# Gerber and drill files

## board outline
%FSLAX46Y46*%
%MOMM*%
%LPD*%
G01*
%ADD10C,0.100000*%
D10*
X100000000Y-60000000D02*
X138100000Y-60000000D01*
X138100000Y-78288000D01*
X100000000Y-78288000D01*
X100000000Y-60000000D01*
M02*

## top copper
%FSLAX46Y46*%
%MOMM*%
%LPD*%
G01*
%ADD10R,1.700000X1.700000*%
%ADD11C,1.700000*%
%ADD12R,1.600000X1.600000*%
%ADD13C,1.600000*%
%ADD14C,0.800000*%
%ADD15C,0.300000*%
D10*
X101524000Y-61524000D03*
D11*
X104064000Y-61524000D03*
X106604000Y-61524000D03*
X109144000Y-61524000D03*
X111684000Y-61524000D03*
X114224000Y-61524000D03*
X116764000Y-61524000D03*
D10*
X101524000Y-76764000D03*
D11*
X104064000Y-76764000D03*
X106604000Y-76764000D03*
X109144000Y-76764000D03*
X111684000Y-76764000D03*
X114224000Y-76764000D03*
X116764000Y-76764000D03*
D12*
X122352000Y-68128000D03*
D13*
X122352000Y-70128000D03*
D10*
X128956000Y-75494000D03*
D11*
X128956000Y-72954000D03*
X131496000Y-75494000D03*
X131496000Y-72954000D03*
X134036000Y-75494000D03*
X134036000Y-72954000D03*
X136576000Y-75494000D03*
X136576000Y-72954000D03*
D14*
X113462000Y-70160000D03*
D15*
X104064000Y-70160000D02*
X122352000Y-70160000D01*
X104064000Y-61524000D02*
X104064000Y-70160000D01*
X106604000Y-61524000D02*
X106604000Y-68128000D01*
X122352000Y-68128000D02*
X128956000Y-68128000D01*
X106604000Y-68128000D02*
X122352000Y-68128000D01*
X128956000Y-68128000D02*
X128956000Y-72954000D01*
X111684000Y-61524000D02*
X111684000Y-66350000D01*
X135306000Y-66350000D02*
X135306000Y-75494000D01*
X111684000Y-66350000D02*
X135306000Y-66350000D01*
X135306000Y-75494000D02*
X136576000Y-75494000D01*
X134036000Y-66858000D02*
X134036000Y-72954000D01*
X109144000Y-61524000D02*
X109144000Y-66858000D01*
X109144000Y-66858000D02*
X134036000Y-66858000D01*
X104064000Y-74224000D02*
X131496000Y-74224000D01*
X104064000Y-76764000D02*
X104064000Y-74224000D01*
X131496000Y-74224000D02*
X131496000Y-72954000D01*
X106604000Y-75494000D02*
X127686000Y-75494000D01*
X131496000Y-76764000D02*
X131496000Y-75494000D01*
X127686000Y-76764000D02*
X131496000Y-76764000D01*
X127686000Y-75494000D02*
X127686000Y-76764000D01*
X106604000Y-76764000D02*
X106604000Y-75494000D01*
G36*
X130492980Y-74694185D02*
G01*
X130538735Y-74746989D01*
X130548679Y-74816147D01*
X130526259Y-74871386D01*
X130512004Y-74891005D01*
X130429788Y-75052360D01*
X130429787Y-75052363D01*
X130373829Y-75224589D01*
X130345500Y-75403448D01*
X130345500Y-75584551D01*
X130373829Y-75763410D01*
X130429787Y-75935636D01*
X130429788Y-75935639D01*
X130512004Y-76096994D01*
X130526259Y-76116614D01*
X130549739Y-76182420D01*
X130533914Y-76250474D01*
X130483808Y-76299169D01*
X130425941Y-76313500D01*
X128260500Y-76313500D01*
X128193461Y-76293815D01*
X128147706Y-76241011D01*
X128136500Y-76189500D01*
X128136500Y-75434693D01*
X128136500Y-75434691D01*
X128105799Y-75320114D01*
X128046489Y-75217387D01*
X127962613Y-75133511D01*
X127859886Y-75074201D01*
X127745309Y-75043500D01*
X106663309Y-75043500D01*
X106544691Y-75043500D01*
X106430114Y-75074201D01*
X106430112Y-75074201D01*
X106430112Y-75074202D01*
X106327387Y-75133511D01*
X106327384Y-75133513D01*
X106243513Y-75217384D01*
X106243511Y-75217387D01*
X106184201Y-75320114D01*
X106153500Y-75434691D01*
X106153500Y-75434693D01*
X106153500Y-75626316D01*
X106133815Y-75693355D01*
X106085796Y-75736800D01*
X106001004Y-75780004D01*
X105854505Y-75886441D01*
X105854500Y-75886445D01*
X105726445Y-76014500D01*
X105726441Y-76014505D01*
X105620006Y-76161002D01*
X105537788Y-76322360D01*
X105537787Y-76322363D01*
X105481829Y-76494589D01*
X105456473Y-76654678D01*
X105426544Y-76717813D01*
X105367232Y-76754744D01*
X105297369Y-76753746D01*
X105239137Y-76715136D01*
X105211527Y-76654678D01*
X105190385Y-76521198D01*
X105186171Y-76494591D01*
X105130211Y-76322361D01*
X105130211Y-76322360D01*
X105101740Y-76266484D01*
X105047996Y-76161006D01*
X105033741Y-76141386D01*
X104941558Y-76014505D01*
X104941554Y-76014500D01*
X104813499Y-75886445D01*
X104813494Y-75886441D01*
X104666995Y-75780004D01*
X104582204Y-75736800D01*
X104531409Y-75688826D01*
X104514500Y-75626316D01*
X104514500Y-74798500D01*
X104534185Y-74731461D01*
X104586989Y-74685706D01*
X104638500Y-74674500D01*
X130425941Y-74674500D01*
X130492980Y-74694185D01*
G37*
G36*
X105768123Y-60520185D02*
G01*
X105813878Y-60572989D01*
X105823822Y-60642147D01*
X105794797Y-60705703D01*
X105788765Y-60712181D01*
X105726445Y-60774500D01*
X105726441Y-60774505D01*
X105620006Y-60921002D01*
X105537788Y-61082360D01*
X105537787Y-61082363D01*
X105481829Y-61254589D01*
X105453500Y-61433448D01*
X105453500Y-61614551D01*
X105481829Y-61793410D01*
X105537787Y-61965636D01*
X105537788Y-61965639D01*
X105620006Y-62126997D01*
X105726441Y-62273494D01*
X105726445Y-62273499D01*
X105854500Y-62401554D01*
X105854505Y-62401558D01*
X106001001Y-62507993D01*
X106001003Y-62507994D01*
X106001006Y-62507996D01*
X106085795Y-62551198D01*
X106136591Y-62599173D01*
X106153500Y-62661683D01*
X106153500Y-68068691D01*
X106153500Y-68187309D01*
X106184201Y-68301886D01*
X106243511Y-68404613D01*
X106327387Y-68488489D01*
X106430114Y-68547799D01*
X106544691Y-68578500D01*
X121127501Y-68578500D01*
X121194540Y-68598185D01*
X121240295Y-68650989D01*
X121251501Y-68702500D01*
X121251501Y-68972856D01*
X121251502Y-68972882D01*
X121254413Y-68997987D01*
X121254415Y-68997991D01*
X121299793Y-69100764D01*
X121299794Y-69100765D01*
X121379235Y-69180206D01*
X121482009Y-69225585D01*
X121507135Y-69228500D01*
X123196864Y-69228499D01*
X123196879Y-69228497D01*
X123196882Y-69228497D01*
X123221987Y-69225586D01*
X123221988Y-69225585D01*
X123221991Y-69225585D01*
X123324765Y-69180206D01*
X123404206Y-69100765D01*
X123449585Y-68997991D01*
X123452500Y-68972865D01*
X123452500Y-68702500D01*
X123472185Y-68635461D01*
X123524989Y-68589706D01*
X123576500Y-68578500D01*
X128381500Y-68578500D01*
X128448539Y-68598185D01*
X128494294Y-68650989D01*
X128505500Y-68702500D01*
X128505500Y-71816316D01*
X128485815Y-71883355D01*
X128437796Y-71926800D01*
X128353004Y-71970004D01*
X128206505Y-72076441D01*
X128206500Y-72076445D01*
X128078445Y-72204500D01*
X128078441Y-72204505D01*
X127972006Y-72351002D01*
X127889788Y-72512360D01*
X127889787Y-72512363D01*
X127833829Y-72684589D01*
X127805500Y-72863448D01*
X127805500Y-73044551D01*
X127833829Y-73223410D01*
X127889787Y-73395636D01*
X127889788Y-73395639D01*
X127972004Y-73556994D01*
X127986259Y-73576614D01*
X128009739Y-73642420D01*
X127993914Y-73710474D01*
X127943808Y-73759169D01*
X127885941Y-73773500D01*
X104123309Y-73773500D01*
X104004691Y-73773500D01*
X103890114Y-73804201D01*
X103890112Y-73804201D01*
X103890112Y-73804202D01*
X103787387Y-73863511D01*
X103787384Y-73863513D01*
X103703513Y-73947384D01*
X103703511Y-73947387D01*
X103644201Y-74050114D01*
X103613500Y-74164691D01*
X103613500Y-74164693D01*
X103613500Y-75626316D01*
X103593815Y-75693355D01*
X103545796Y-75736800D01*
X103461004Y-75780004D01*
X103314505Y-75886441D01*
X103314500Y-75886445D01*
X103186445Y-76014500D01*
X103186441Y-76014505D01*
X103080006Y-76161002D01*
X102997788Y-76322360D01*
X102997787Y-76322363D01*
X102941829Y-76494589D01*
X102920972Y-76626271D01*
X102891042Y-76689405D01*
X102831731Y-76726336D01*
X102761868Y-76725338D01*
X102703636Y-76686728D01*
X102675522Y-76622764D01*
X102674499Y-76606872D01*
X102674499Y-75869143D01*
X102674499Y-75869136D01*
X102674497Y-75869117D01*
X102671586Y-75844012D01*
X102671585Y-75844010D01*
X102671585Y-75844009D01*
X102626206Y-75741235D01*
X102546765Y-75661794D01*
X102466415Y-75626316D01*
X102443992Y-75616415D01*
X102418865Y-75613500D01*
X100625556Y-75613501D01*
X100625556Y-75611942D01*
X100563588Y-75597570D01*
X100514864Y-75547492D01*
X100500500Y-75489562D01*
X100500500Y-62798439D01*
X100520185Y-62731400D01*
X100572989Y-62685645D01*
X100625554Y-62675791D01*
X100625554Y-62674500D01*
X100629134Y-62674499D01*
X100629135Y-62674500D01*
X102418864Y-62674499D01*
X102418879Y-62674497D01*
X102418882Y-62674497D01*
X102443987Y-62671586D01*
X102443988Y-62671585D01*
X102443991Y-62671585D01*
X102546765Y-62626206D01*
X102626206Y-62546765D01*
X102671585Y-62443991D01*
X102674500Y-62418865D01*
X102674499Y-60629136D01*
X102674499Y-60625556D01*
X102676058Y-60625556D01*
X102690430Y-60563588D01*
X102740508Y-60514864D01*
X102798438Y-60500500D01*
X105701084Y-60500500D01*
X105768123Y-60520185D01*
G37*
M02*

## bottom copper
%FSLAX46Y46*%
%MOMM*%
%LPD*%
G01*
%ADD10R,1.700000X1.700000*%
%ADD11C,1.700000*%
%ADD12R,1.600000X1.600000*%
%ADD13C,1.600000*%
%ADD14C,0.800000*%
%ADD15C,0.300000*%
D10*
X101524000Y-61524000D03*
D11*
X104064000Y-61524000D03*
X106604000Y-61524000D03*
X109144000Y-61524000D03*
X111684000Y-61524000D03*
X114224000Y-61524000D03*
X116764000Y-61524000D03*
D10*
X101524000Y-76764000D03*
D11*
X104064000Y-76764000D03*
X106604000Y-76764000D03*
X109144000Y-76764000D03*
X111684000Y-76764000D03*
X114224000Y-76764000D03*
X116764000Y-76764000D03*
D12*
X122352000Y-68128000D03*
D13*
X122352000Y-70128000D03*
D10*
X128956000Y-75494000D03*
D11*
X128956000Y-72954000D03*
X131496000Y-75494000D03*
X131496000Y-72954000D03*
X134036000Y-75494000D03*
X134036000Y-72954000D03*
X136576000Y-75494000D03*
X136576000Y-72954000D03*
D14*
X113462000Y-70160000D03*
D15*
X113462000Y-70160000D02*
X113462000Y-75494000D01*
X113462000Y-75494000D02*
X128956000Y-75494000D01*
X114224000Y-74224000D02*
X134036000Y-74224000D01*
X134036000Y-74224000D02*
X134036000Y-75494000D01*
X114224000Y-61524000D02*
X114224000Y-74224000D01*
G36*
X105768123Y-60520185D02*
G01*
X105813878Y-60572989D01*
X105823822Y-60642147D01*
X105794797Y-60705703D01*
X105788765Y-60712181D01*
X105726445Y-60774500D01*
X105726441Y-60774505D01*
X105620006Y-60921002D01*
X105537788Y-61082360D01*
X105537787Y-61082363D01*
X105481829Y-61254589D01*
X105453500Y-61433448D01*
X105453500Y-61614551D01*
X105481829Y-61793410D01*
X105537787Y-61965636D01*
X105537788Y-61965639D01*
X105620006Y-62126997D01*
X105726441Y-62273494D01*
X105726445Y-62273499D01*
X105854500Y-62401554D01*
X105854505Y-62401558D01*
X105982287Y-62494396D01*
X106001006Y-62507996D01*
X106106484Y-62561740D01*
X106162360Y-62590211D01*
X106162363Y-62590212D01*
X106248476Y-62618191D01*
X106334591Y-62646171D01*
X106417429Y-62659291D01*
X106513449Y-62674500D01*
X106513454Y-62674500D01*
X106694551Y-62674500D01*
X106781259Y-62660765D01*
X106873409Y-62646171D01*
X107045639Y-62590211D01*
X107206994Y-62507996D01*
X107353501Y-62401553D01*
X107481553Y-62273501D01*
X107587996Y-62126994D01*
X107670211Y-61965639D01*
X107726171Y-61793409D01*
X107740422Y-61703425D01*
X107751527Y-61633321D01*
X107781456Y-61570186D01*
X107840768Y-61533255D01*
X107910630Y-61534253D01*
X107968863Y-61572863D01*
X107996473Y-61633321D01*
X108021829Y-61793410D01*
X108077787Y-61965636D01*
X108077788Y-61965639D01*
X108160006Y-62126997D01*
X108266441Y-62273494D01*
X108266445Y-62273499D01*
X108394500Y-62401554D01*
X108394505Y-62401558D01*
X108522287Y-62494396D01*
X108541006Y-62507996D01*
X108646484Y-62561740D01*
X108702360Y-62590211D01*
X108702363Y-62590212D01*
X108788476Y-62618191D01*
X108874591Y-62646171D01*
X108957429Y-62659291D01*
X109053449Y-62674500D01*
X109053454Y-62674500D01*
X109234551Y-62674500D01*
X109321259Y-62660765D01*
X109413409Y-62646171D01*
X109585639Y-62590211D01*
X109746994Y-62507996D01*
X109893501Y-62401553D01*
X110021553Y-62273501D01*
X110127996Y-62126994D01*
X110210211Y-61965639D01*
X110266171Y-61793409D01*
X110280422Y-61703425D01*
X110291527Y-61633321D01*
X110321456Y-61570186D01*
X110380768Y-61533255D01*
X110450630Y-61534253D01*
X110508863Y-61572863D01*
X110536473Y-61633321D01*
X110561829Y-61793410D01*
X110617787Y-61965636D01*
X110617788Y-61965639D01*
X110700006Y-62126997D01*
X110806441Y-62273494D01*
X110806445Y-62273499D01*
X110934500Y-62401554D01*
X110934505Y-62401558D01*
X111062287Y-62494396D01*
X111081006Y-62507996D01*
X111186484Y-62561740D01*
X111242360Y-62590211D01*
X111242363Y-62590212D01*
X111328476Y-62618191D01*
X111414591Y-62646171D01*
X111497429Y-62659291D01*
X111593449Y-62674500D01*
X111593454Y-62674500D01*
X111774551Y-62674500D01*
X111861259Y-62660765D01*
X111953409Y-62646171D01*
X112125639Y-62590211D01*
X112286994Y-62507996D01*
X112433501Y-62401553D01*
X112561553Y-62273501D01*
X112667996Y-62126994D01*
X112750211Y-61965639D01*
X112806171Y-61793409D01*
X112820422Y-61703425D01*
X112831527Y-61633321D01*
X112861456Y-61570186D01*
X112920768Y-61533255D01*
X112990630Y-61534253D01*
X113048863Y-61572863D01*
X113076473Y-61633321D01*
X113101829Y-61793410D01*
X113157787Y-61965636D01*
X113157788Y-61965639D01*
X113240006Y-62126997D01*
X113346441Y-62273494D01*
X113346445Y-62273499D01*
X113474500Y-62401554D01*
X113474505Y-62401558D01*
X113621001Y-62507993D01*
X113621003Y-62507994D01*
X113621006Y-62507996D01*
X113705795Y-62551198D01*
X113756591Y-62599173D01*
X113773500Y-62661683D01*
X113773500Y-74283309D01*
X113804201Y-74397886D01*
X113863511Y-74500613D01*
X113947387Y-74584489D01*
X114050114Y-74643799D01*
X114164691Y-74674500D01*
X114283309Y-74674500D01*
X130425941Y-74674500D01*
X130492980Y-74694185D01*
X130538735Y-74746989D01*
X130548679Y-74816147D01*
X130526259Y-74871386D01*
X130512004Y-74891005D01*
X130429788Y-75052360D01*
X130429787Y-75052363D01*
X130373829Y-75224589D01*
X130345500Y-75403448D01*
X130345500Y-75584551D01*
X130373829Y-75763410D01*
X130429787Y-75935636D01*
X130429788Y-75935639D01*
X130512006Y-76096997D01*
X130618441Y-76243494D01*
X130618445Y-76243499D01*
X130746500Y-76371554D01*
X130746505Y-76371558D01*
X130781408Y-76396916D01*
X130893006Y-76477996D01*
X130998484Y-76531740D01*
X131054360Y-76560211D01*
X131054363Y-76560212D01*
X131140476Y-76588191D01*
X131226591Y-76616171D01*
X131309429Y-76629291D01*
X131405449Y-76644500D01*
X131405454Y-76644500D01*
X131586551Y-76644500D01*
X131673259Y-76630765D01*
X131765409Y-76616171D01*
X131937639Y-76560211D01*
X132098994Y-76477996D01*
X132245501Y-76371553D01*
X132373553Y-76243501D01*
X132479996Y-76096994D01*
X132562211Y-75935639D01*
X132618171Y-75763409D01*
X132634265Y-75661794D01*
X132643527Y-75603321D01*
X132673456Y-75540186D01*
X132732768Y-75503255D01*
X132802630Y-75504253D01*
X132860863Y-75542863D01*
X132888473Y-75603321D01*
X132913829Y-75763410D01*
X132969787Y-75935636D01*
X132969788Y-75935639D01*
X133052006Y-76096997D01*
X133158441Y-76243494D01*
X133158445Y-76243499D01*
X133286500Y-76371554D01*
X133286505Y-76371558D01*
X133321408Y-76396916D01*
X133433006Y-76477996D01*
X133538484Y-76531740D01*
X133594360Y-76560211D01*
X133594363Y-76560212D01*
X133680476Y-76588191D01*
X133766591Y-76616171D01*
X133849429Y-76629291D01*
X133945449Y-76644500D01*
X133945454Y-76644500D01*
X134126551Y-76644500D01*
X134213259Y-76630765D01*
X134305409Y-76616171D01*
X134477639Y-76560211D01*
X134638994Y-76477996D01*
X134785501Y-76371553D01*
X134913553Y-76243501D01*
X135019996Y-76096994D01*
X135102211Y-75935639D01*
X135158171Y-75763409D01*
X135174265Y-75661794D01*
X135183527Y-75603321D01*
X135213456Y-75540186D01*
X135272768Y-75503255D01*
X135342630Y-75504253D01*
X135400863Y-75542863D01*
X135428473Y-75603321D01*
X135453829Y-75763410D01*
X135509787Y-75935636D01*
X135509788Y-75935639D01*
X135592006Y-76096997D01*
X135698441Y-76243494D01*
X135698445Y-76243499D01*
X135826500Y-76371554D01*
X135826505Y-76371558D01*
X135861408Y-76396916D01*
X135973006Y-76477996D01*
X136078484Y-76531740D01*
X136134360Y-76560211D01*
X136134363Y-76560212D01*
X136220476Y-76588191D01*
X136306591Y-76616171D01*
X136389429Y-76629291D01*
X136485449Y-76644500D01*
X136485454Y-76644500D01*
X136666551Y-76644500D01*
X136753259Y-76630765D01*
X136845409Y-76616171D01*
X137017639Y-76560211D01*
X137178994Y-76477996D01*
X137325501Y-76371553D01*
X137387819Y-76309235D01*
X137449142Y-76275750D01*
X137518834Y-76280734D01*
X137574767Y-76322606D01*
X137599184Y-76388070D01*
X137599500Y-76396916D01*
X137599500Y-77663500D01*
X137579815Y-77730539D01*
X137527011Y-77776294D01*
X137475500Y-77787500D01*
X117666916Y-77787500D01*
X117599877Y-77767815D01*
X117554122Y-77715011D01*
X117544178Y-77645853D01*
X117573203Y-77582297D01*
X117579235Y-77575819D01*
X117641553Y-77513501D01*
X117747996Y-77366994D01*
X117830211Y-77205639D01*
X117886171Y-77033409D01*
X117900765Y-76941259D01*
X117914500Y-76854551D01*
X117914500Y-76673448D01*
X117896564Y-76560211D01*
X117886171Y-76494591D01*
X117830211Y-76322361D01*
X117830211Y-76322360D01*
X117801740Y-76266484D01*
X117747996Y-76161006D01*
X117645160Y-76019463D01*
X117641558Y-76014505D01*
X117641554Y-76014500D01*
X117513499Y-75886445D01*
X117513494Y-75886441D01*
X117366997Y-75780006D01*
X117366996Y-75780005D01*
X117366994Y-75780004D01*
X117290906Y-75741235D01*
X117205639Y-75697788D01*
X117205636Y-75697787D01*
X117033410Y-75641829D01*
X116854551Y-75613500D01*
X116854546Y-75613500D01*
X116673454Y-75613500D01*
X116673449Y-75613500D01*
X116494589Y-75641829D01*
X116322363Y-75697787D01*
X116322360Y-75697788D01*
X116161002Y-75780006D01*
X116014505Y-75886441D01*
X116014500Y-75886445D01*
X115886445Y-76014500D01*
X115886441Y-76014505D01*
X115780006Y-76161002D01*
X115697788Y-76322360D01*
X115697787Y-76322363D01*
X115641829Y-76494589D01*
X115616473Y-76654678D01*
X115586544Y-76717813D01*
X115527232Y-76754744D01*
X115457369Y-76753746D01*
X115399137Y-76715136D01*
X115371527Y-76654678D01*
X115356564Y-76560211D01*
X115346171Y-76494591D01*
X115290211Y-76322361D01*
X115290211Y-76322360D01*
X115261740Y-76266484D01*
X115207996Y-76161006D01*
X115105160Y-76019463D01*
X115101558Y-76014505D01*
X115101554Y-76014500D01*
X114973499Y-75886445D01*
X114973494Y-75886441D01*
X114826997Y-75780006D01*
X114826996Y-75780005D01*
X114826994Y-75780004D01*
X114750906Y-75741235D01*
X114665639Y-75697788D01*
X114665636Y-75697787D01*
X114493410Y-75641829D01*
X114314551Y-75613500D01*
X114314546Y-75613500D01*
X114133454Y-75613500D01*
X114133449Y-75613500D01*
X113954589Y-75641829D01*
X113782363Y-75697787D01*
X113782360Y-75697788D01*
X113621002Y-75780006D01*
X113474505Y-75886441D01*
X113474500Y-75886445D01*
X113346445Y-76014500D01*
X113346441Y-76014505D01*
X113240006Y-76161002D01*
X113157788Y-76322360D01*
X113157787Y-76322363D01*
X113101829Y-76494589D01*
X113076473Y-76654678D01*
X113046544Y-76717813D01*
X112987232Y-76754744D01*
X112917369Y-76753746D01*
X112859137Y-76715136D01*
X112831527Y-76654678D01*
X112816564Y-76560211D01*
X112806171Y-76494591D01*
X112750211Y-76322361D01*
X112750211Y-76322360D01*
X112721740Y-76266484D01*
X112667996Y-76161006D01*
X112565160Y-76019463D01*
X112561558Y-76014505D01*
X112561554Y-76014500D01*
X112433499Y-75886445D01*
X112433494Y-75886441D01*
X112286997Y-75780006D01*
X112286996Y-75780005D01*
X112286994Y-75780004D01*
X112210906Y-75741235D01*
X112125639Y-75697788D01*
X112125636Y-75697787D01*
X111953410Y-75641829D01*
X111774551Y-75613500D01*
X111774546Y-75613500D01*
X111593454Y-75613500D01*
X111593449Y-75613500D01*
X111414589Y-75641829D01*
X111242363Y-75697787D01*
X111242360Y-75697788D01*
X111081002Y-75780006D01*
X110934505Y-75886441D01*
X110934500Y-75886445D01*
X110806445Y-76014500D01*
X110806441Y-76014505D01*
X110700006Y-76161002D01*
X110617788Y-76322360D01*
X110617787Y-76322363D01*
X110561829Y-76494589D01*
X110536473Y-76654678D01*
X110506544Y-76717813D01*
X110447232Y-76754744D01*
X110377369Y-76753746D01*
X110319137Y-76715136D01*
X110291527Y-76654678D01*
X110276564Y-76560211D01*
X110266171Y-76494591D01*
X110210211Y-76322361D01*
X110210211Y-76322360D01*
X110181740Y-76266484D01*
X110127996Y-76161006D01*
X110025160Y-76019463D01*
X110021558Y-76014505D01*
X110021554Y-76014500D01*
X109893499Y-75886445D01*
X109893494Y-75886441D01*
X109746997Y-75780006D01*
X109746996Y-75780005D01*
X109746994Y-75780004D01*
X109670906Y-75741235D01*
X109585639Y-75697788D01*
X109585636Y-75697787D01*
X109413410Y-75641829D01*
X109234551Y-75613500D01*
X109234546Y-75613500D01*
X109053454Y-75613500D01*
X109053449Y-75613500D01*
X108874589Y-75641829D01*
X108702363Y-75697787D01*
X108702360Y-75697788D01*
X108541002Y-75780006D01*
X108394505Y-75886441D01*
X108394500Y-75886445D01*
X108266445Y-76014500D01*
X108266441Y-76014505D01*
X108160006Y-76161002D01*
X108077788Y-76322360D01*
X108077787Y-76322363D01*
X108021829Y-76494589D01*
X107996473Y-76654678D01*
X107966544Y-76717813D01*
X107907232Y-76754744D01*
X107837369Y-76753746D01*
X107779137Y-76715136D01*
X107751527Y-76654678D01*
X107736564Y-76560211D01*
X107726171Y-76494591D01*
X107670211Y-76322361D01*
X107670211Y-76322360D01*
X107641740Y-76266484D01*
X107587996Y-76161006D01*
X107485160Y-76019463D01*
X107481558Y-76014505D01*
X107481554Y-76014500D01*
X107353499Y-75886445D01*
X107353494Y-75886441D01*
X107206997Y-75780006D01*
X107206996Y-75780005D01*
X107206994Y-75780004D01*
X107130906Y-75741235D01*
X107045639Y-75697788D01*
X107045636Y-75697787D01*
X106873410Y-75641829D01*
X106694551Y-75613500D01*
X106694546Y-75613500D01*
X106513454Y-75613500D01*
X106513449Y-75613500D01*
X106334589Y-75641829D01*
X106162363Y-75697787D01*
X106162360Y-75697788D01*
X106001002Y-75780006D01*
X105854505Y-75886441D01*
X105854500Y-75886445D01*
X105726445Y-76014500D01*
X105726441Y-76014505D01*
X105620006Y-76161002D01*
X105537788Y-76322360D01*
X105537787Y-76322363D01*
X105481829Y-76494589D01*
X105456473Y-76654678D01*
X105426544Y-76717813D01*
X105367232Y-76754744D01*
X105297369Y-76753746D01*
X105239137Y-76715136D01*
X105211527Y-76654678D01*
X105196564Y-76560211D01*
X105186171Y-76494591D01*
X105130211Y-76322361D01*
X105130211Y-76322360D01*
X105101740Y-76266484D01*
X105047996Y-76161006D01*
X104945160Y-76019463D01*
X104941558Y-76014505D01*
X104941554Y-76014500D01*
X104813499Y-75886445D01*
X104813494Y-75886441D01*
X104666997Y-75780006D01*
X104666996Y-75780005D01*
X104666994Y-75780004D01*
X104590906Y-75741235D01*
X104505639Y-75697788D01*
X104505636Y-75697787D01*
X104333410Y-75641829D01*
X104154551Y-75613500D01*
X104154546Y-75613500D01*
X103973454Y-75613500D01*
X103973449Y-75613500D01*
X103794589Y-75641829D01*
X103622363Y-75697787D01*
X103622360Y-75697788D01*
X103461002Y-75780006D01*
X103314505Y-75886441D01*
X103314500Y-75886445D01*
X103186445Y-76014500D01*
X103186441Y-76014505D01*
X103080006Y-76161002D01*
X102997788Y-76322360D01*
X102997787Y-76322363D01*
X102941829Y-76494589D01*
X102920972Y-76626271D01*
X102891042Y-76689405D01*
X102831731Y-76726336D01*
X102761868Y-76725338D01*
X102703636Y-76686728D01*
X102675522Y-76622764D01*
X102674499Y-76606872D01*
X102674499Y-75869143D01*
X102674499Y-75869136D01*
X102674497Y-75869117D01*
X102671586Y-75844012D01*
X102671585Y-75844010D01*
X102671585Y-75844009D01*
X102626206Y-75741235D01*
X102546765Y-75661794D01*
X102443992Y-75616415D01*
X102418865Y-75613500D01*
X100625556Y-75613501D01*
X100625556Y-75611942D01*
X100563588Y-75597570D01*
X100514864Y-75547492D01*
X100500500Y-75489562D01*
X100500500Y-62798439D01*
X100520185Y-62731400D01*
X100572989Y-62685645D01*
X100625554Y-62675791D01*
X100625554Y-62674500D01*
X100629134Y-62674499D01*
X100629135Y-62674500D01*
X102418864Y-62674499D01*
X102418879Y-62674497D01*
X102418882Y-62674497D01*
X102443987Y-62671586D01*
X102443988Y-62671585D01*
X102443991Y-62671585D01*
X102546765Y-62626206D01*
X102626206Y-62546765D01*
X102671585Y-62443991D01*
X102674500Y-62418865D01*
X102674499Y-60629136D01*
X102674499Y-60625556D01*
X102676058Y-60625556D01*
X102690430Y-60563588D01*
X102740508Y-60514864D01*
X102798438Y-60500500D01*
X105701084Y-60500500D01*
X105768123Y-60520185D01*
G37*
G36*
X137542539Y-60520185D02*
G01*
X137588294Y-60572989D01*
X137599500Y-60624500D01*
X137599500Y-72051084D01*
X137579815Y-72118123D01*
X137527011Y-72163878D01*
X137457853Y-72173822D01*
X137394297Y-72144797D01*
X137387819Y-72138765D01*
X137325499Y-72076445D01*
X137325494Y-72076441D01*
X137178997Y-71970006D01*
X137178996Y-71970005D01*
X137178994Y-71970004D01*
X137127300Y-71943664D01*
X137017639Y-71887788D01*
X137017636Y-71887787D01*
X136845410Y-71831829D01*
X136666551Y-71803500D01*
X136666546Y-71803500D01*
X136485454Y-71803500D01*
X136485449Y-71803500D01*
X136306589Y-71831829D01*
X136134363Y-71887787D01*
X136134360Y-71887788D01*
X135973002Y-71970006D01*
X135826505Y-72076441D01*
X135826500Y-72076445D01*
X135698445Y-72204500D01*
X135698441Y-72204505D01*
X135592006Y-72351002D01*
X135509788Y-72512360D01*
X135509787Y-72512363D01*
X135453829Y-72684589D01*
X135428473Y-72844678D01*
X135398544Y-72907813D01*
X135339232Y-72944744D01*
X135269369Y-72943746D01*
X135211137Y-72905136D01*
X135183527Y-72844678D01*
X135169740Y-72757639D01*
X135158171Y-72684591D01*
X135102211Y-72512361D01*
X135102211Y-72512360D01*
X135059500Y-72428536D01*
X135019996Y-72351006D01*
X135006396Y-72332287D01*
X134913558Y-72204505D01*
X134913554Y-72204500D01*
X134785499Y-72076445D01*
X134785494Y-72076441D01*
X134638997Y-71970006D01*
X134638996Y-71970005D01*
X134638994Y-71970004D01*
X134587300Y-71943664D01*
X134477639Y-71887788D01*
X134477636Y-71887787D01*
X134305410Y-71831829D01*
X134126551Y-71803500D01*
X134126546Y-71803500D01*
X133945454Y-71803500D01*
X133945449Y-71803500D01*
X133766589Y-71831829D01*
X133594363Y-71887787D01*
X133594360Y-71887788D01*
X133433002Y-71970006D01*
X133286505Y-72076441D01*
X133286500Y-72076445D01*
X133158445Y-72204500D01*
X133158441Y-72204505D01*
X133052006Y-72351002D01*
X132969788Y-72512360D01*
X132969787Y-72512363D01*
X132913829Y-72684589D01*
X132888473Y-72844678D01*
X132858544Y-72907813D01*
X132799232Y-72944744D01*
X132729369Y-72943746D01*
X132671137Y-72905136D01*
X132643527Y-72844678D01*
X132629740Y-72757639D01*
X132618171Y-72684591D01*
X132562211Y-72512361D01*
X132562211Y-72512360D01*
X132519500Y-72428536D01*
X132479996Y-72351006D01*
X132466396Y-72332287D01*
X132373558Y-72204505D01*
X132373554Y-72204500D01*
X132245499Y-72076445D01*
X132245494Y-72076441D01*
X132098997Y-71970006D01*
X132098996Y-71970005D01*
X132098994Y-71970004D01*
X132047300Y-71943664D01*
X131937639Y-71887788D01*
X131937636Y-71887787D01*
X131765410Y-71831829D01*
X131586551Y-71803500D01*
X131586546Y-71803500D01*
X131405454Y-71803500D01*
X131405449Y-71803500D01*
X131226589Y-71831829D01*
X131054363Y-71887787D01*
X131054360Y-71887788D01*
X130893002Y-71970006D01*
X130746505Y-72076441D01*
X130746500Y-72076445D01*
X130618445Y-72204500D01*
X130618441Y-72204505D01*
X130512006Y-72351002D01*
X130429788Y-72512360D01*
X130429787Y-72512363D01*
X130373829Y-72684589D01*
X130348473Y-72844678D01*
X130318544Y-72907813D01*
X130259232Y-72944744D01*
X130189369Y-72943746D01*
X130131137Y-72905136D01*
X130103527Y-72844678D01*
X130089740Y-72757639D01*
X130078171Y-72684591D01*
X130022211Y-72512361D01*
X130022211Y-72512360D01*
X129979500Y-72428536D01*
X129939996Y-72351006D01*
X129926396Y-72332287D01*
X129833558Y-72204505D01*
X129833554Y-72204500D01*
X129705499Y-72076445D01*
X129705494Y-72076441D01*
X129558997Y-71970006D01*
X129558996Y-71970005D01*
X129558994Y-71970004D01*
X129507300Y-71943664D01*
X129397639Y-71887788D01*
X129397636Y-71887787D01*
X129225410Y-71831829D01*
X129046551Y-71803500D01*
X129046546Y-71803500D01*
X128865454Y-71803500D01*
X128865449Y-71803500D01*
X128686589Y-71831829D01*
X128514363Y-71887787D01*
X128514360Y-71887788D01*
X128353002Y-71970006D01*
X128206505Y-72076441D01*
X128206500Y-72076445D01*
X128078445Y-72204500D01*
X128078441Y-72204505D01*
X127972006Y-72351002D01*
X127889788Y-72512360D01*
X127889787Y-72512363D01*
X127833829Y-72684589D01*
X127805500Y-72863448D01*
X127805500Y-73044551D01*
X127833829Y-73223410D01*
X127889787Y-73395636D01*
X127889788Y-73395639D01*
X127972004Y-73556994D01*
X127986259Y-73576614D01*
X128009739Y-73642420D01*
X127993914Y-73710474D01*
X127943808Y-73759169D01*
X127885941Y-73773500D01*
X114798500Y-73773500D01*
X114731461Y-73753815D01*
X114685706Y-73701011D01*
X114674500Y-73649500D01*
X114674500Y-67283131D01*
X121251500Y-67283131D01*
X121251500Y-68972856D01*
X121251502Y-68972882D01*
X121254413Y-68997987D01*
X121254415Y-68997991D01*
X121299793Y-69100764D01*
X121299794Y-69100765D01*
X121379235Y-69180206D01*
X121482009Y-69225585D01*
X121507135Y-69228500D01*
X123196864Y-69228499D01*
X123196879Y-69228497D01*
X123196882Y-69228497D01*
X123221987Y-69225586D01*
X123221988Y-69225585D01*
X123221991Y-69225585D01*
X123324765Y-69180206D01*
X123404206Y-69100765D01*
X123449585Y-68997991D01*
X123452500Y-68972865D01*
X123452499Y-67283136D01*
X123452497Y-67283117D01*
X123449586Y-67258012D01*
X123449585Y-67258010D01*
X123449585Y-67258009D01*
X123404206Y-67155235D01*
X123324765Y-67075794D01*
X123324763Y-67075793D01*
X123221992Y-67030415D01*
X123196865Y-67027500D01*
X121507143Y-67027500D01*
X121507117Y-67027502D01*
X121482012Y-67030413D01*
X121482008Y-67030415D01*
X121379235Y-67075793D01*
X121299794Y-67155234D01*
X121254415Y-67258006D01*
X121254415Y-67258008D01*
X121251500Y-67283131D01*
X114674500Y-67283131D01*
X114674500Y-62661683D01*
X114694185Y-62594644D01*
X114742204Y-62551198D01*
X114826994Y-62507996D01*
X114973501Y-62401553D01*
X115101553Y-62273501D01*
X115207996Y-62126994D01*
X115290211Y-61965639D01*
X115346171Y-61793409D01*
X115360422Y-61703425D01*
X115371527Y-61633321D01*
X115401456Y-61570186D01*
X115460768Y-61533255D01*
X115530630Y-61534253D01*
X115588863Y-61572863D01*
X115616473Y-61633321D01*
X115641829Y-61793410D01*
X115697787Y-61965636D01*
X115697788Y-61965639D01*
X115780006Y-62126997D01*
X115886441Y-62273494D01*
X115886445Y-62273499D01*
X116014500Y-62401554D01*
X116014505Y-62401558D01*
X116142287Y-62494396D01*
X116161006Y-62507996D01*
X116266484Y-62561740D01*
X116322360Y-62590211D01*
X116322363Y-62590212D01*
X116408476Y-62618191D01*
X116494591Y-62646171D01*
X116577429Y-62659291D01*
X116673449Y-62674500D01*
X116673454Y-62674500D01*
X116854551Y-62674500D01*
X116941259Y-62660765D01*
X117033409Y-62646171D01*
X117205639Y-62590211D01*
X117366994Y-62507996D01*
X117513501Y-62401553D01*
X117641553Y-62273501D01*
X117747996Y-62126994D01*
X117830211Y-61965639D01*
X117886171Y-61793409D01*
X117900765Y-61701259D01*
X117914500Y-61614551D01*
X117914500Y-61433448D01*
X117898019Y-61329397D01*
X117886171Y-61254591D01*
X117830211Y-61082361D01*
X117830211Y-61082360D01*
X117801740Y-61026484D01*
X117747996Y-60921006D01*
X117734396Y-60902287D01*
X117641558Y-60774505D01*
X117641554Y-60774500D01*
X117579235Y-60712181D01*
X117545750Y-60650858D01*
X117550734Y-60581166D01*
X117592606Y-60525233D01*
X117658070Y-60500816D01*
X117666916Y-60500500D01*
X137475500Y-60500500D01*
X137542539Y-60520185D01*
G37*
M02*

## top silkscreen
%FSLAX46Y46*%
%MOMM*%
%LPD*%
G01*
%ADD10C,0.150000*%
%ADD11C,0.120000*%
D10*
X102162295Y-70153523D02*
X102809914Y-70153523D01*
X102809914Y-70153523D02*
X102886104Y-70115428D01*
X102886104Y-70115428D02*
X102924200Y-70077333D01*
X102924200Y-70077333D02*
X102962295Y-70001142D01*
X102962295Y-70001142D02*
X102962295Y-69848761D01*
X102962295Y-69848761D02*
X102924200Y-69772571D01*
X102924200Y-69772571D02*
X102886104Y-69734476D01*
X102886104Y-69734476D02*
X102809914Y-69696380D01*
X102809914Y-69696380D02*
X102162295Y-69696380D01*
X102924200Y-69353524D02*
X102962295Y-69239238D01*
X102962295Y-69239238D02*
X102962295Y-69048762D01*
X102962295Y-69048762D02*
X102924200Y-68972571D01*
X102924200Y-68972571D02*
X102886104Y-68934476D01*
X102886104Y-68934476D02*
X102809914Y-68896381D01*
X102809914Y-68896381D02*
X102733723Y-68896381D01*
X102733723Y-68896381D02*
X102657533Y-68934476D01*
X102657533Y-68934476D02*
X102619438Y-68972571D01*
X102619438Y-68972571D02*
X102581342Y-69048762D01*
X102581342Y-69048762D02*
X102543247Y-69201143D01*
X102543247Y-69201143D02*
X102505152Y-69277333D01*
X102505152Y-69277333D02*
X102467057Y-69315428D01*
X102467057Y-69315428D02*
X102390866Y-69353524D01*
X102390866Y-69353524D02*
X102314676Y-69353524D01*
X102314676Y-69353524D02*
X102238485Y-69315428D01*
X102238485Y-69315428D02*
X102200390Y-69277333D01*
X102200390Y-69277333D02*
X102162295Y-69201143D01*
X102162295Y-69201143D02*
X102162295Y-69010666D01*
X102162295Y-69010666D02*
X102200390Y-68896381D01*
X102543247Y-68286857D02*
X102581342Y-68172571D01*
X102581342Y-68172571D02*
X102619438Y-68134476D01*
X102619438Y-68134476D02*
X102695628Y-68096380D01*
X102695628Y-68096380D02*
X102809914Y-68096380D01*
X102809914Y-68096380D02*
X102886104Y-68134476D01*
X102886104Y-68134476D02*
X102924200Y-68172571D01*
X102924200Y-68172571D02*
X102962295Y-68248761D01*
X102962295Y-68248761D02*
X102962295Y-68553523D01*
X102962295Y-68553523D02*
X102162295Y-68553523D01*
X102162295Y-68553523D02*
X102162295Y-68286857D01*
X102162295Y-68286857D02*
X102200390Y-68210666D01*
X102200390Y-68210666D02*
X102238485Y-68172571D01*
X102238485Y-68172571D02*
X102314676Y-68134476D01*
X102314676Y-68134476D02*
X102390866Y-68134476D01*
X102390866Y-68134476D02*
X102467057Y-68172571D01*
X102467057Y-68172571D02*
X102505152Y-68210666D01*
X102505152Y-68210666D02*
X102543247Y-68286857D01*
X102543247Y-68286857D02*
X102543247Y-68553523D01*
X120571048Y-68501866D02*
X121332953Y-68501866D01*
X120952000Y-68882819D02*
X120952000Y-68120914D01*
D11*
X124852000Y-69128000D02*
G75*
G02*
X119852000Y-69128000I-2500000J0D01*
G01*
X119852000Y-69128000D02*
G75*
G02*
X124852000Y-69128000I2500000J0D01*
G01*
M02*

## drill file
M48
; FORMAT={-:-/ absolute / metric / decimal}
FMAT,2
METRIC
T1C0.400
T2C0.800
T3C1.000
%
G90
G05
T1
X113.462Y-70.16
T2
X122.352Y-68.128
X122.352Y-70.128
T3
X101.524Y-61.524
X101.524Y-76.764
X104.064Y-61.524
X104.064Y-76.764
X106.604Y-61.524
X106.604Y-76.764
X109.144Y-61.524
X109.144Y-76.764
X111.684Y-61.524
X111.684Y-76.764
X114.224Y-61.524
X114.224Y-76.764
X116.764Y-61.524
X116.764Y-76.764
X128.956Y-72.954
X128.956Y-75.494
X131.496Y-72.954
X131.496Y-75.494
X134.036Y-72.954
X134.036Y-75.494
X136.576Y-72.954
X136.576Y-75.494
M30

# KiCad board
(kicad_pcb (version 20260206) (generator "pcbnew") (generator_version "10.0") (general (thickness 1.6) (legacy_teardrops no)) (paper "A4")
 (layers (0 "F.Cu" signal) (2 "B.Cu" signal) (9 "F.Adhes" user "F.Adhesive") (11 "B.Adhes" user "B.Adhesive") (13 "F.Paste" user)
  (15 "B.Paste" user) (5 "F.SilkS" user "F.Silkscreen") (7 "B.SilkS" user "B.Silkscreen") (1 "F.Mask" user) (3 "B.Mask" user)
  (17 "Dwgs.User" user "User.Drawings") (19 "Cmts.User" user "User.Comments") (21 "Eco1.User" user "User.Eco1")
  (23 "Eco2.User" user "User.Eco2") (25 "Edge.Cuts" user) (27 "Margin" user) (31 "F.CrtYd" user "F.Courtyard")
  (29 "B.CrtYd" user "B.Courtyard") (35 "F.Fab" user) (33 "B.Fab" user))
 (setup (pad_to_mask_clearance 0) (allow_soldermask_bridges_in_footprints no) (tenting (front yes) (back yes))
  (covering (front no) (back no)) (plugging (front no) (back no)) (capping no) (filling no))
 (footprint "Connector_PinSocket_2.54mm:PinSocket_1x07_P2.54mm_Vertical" (layer "F.Cu") (at 101.524 61.524)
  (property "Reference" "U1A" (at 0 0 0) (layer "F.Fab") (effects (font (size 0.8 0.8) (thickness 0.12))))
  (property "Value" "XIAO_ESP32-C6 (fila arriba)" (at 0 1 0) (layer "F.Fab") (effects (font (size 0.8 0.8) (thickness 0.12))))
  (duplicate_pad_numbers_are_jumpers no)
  (pad "1" thru_hole rect (at 0 0) (size 1.7 1.7) (drill 1) (layers "*.Cu" "*.Mask") (remove_unused_layers no))
  (pad "2" thru_hole circle (at 2.54 0) (size 1.7 1.7) (drill 1) (layers "*.Cu" "*.Mask") (remove_unused_layers no) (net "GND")
   (zone_connect 2))
  (pad "3" thru_hole circle (at 5.08 0) (size 1.7 1.7) (drill 1) (layers "*.Cu" "*.Mask") (remove_unused_layers no) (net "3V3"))
  (pad "4" thru_hole circle (at 7.62 0) (size 1.7 1.7) (drill 1) (layers "*.Cu" "*.Mask") (remove_unused_layers no) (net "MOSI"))
  (pad "5" thru_hole circle (at 10.16 0) (size 1.7 1.7) (drill 1) (layers "*.Cu" "*.Mask") (remove_unused_layers no) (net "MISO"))
  (pad "6" thru_hole circle (at 12.7 0) (size 1.7 1.7) (drill 1) (layers "*.Cu" "*.Mask") (remove_unused_layers no) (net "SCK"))
  (pad "7" thru_hole circle (at 15.24 0) (size 1.7 1.7) (drill 1) (layers "*.Cu" "*.Mask") (remove_unused_layers no)))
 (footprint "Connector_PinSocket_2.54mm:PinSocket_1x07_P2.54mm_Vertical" (layer "F.Cu") (at 101.524 76.764)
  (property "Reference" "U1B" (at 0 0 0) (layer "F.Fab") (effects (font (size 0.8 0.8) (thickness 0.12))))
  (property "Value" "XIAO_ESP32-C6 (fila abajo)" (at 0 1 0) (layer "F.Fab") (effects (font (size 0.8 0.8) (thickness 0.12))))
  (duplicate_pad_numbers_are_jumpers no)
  (pad "1" thru_hole rect (at 0 0) (size 1.7 1.7) (drill 1) (layers "*.Cu" "*.Mask") (remove_unused_layers no))
  (pad "2" thru_hole circle (at 2.54 0) (size 1.7 1.7) (drill 1) (layers "*.Cu" "*.Mask") (remove_unused_layers no) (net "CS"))
  (pad "3" thru_hole circle (at 5.08 0) (size 1.7 1.7) (drill 1) (layers "*.Cu" "*.Mask") (remove_unused_layers no) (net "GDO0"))
  (pad "4" thru_hole circle (at 7.62 0) (size 1.7 1.7) (drill 1) (layers "*.Cu" "*.Mask") (remove_unused_layers no))
  (pad "5" thru_hole circle (at 10.16 0) (size 1.7 1.7) (drill 1) (layers "*.Cu" "*.Mask") (remove_unused_layers no))
  (pad "6" thru_hole circle (at 12.7 0) (size 1.7 1.7) (drill 1) (layers "*.Cu" "*.Mask") (remove_unused_layers no))
  (pad "7" thru_hole circle (at 15.24 0) (size 1.7 1.7) (drill 1) (layers "*.Cu" "*.Mask") (remove_unused_layers no)))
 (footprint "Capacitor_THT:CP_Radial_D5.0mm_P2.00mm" (layer "F.Cu") (at 122.352 68.128)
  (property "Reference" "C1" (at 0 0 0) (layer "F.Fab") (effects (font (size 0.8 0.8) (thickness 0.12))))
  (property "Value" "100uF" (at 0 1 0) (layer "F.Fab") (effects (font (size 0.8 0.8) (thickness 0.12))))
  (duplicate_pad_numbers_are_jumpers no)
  (fp_circle (center 0 1) (end 2.5 1) (stroke (width 0.12) (type solid)) (fill no) (layer "F.SilkS"))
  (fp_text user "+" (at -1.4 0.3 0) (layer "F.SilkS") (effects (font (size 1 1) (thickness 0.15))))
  (pad "1" thru_hole rect (at 0 0) (size 1.6 1.6) (drill 0.8) (layers "*.Cu" "*.Mask") (remove_unused_layers no) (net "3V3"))
  (pad "2" thru_hole circle (at 0 2) (size 1.6 1.6) (drill 0.8) (layers "*.Cu" "*.Mask") (remove_unused_layers no) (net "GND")
   (zone_connect 2)))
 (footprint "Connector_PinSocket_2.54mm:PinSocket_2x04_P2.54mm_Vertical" (layer "F.Cu") (at 128.956 75.494)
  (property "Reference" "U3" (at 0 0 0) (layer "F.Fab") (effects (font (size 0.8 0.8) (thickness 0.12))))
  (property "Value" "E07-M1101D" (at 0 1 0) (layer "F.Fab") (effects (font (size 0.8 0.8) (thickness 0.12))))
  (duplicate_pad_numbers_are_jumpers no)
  (pad "1" thru_hole rect (at 0 0) (size 1.7 1.7) (drill 1) (layers "*.Cu" "*.Mask") (remove_unused_layers no) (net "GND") (zone_connect 2))
  (pad "2" thru_hole circle (at 0 -2.54) (size 1.7 1.7) (drill 1) (layers "*.Cu" "*.Mask") (remove_unused_layers no) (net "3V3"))
  (pad "3" thru_hole circle (at 2.54 0) (size 1.7 1.7) (drill 1) (layers "*.Cu" "*.Mask") (remove_unused_layers no) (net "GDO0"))
  (pad "4" thru_hole circle (at 2.54 -2.54) (size 1.7 1.7) (drill 1) (layers "*.Cu" "*.Mask") (remove_unused_layers no) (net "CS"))
  (pad "5" thru_hole circle (at 5.08 0) (size 1.7 1.7) (drill 1) (layers "*.Cu" "*.Mask") (remove_unused_layers no) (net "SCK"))
  (pad "6" thru_hole circle (at 5.08 -2.54) (size 1.7 1.7) (drill 1) (layers "*.Cu" "*.Mask") (remove_unused_layers no) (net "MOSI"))
  (pad "7" thru_hole circle (at 7.62 0) (size 1.7 1.7) (drill 1) (layers "*.Cu" "*.Mask") (remove_unused_layers no) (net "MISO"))
  (pad "8" thru_hole circle (at 7.62 -2.54) (size 1.7 1.7) (drill 1) (layers "*.Cu" "*.Mask") (remove_unused_layers no)))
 (gr_rect (start 100 60) (end 138.1 78.288) (stroke (width 0.1) (type default)) (fill no) (layer "Edge.Cuts"))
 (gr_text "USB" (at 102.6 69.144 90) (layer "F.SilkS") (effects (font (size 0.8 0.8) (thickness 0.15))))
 (segment (start 104.064 70.16) (end 122.352 70.16) (width 0.3) (layer "F.Cu") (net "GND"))
 (segment (start 104.064 61.524) (end 104.064 70.16) (width 0.3) (layer "F.Cu") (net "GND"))
 (via (at 113.462 70.16) (size 0.8) (drill 0.4) (layers "F.Cu" "B.Cu") (capping no) (covering (front no) (back no))
  (plugging (front no) (back no)) (filling no) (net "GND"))
 (segment (start 113.462 70.16) (end 113.462 75.494) (width 0.3) (layer "B.Cu") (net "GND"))
 (segment (start 113.462 75.494) (end 128.956 75.494) (width 0.3) (layer "B.Cu") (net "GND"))
 (segment (start 106.604 61.524) (end 106.604 68.128) (width 0.3) (layer "F.Cu") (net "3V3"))
 (segment (start 122.352 68.128) (end 128.956 68.128) (width 0.3) (layer "F.Cu") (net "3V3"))
 (segment (start 106.604 68.128) (end 122.352 68.128) (width 0.3) (layer "F.Cu") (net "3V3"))
 (segment (start 128.956 68.128) (end 128.956 72.954) (width 0.3) (layer "F.Cu") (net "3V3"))
 (segment (start 114.224 74.224) (end 134.036 74.224) (width 0.3) (layer "B.Cu") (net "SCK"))
 (segment (start 134.036 74.224) (end 134.036 75.494) (width 0.3) (layer "B.Cu") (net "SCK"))
 (segment (start 114.224 61.524) (end 114.224 74.224) (width 0.3) (layer "B.Cu") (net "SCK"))
 (segment (start 111.684 61.524) (end 111.684 66.35) (width 0.3) (layer "F.Cu") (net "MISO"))
 (segment (start 135.306 66.35) (end 135.306 75.494) (width 0.3) (layer "F.Cu") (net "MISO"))
 (segment (start 111.684 66.35) (end 135.306 66.35) (width 0.3) (layer "F.Cu") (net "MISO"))
 (segment (start 135.306 75.494) (end 136.576 75.494) (width 0.3) (layer "F.Cu") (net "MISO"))
 (segment (start 134.036 66.858) (end 134.036 72.954) (width 0.3) (layer "F.Cu") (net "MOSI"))
 (segment (start 109.144 61.524) (end 109.144 66.858) (width 0.3) (layer "F.Cu") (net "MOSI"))
 (segment (start 109.144 66.858) (end 134.036 66.858) (width 0.3) (layer "F.Cu") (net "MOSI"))
 (segment (start 104.064 74.224) (end 131.496 74.224) (width 0.3) (layer "F.Cu") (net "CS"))
 (segment (start 104.064 76.764) (end 104.064 74.224) (width 0.3) (layer "F.Cu") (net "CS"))
 (segment (start 131.496 74.224) (end 131.496 72.954) (width 0.3) (layer "F.Cu") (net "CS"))
 (segment (start 106.604 75.494) (end 127.686 75.494) (width 0.3) (layer "F.Cu") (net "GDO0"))
 (segment (start 131.496 76.764) (end 131.496 75.494) (width 0.3) (layer "F.Cu") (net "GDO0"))
 (segment (start 127.686 76.764) (end 131.496 76.764) (width 0.3) (layer "F.Cu") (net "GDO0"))
 (segment (start 127.686 75.494) (end 127.686 76.764) (width 0.3) (layer "F.Cu") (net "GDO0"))
 (segment (start 106.604 76.764) (end 106.604 75.494) (width 0.3) (layer "F.Cu") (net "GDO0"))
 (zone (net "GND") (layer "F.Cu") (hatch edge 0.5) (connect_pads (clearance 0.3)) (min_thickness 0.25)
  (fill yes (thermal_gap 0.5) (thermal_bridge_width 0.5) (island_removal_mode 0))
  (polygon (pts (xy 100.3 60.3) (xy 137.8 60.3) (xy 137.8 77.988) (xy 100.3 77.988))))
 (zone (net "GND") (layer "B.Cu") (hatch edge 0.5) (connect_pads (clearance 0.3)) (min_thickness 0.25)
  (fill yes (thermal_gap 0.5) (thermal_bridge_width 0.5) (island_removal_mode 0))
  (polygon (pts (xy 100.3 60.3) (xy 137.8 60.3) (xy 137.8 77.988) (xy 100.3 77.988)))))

